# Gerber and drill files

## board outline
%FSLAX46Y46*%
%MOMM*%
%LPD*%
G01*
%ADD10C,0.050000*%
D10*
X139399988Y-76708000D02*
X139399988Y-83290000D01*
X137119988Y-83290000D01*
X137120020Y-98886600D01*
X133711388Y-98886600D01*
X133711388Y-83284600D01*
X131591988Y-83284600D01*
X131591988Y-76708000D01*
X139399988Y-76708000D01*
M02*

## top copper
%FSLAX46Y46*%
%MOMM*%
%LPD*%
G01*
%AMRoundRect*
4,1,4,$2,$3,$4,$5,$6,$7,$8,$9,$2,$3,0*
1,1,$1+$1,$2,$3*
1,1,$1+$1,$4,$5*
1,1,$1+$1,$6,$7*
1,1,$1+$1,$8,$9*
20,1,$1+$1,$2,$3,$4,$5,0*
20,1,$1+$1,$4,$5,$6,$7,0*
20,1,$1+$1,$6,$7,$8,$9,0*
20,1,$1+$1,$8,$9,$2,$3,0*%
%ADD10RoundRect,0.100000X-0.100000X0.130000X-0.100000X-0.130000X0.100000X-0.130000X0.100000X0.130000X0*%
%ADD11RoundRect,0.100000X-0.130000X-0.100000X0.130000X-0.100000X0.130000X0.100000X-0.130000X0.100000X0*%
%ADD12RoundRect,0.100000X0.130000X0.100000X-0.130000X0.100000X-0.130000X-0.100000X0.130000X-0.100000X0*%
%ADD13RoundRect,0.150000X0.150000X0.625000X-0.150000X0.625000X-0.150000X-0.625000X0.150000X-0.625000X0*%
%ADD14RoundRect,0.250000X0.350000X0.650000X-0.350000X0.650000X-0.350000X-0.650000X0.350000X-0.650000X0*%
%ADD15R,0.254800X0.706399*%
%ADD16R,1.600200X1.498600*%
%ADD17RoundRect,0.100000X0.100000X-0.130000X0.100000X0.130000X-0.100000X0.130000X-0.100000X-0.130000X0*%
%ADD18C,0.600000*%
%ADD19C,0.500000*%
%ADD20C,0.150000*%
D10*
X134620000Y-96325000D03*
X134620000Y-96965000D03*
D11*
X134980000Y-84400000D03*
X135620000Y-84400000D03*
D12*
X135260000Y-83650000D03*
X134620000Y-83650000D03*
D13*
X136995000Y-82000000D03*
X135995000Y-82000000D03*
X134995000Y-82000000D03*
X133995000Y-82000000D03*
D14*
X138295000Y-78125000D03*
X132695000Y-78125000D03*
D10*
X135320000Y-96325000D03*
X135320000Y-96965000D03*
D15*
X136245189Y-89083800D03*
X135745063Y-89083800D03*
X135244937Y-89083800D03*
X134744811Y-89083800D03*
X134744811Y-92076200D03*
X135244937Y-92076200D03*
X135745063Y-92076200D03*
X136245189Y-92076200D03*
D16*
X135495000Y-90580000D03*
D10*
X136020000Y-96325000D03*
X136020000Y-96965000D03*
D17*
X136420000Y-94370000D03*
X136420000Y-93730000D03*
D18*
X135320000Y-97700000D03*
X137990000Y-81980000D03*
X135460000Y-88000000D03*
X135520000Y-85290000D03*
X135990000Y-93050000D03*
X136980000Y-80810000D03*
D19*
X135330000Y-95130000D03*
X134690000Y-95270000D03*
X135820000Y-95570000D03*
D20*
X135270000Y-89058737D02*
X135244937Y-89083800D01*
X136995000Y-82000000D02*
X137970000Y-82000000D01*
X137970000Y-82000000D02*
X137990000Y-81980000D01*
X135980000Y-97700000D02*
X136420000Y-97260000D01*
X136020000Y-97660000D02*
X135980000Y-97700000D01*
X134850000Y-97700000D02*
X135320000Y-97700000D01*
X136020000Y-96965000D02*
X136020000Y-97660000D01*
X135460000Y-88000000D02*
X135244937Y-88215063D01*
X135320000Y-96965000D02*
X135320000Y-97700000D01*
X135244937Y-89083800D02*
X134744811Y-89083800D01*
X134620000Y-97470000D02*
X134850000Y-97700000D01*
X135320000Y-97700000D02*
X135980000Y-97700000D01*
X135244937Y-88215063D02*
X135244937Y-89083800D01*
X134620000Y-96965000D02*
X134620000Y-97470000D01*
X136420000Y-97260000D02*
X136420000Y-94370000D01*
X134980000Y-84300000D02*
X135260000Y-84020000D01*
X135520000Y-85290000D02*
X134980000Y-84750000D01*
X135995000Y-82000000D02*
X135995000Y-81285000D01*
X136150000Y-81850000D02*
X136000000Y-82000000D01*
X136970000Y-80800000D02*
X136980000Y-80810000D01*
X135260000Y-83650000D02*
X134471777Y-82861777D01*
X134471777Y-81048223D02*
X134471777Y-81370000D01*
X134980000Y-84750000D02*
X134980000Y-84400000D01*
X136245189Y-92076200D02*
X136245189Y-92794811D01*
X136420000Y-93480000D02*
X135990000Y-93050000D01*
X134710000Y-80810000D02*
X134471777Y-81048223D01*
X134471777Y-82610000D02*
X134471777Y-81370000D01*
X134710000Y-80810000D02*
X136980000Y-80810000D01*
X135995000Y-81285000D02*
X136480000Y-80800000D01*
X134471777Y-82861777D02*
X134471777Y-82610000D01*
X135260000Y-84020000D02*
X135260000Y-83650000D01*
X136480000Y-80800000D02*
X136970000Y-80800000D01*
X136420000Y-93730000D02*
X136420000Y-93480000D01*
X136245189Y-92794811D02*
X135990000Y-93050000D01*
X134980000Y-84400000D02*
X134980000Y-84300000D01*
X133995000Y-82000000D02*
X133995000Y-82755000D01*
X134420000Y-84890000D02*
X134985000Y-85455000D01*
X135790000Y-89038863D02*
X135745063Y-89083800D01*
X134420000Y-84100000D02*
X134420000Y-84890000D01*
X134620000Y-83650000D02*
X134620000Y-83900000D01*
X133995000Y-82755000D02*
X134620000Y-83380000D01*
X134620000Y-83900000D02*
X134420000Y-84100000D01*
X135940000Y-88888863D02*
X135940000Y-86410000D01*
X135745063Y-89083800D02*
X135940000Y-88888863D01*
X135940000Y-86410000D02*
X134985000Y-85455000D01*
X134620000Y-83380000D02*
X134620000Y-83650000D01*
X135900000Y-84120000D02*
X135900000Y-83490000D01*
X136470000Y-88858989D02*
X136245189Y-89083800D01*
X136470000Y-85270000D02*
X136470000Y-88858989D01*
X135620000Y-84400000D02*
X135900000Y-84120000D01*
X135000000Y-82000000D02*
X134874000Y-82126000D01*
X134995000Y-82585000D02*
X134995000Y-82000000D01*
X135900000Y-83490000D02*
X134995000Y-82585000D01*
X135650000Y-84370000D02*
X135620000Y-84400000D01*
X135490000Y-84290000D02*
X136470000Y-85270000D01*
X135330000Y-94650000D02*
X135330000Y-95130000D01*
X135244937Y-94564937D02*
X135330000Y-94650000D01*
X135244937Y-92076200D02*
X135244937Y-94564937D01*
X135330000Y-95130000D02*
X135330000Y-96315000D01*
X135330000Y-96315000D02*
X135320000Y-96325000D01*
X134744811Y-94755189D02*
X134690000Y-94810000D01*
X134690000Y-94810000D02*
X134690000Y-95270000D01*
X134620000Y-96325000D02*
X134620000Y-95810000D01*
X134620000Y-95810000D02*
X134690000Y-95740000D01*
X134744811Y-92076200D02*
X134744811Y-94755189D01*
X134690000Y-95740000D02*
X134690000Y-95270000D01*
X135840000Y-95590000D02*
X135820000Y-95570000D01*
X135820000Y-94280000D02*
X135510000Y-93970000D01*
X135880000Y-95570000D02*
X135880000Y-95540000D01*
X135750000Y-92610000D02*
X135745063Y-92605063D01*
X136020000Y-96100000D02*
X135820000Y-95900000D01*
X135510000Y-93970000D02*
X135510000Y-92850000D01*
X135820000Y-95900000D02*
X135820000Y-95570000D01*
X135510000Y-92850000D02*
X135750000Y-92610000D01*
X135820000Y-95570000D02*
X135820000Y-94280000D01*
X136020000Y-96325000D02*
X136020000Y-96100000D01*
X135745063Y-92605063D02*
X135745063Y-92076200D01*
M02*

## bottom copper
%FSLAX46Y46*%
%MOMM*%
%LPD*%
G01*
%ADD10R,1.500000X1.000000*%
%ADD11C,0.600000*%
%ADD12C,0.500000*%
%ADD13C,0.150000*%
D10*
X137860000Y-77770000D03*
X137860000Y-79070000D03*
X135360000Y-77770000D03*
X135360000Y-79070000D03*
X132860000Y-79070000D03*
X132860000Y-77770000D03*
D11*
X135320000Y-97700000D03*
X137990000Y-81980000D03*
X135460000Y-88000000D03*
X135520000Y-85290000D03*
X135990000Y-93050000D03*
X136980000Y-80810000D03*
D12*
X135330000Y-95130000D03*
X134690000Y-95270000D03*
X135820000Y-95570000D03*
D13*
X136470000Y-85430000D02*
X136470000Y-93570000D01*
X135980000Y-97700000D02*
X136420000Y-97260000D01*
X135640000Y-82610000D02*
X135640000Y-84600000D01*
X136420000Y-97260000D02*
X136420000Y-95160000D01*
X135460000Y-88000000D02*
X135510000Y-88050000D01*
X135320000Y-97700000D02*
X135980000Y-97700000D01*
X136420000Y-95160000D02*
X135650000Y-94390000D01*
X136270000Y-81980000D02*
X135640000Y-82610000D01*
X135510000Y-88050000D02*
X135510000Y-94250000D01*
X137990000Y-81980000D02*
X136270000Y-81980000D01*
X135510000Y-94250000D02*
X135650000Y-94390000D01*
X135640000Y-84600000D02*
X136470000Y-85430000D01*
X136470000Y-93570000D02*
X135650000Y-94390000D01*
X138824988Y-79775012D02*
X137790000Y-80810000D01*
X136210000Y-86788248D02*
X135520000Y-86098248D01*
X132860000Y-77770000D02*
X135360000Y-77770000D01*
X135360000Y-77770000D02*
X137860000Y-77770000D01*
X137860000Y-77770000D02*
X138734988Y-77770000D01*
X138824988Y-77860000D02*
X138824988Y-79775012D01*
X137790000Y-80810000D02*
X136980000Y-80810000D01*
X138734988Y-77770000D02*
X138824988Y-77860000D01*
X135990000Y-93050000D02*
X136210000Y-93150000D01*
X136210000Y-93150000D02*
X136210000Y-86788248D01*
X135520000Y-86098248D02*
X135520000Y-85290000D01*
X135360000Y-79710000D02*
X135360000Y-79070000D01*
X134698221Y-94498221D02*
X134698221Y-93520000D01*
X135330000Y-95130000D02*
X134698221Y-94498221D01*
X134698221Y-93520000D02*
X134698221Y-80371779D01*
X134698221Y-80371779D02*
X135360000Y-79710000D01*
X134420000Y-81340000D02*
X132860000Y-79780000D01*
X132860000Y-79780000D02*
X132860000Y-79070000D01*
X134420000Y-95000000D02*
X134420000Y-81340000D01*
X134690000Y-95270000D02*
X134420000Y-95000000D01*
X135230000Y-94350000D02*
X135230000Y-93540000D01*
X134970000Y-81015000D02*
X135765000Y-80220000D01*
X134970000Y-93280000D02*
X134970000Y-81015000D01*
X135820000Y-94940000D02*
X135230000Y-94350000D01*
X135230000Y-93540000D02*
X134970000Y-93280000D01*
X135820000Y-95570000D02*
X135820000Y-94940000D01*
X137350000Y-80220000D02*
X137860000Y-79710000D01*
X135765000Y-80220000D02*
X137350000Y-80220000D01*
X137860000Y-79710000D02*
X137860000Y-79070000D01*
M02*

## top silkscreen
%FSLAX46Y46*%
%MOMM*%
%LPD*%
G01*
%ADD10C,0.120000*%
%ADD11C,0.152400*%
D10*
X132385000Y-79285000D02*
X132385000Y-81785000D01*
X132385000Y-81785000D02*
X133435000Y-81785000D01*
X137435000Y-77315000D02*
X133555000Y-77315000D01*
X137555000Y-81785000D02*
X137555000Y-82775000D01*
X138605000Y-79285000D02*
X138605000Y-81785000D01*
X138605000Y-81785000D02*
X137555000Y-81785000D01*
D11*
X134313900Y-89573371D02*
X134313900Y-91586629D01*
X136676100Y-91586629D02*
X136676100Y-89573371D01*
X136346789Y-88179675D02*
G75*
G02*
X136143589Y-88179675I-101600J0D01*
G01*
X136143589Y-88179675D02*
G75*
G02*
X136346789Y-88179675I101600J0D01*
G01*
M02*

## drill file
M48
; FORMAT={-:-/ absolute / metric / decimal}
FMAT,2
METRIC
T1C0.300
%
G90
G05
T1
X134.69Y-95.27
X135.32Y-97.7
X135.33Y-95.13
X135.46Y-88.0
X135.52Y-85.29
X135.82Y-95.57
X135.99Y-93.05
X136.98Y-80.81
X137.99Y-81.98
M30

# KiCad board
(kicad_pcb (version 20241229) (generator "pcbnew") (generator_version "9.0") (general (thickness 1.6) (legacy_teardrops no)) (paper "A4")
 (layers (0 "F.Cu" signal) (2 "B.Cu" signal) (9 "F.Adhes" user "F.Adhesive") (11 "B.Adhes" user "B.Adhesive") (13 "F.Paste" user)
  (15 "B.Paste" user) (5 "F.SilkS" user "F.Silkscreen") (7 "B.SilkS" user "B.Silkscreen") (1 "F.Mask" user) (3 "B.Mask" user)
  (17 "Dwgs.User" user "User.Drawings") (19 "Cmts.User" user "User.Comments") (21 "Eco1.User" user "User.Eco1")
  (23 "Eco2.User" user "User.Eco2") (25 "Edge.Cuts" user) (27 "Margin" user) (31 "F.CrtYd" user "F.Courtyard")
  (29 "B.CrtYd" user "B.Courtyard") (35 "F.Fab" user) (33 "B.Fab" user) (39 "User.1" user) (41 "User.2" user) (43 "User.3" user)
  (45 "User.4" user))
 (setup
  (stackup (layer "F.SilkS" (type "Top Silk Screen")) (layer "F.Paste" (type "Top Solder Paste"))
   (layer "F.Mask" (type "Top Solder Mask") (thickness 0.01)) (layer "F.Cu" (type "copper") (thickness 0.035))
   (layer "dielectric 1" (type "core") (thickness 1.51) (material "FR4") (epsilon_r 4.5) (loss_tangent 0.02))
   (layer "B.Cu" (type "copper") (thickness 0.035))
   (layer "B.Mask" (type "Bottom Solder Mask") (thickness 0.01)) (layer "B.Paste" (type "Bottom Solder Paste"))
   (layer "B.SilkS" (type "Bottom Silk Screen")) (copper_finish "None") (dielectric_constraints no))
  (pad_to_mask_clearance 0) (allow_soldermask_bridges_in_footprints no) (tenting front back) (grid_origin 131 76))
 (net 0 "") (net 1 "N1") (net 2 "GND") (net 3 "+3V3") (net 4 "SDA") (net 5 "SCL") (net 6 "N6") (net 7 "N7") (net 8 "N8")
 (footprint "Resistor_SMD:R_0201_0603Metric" (layer "F.Cu") (at 134.62 96.645 -90)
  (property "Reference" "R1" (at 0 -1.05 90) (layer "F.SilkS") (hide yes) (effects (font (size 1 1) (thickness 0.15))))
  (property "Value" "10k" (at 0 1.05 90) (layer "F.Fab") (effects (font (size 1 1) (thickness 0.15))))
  (pad "" smd roundrect (at -0.345 0 270) (size 0.318 0.36) (layers "F.Paste") (roundrect_rratio 0.25))
  (pad "" smd roundrect (at 0.345 0 270) (size 0.318 0.36) (layers "F.Paste") (roundrect_rratio 0.25))
  (pad "1" smd roundrect (at -0.32 0 270) (size 0.46 0.4) (layers "F.Cu" "F.Mask") (roundrect_rratio 0.25) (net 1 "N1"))
  (pad "2" smd roundrect (at 0.32 0 270) (size 0.46 0.4) (layers "F.Cu" "F.Mask") (roundrect_rratio 0.25) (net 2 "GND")))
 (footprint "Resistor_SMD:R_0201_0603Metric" (layer "F.Cu") (at 135.3 84.4)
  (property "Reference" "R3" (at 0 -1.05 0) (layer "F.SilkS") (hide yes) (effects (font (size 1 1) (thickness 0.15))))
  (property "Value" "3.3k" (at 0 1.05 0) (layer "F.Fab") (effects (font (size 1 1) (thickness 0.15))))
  (pad "" smd roundrect (at -0.345 0) (size 0.318 0.36) (layers "F.Paste") (roundrect_rratio 0.25))
  (pad "" smd roundrect (at 0.345 0) (size 0.318 0.36) (layers "F.Paste") (roundrect_rratio 0.25))
  (pad "1" smd roundrect (at -0.32 0) (size 0.46 0.4) (layers "F.Cu" "F.Mask") (roundrect_rratio 0.25) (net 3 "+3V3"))
  (pad "2" smd roundrect (at 0.32 0) (size 0.46 0.4) (layers "F.Cu" "F.Mask") (roundrect_rratio 0.25) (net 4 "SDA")))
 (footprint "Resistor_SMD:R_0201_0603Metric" (layer "F.Cu") (at 134.94 83.65 180)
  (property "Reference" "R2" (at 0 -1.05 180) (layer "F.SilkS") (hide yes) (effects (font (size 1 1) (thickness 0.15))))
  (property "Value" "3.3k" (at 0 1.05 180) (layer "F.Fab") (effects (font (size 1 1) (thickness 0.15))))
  (pad "" smd roundrect (at -0.345 0 180) (size 0.318 0.36) (layers "F.Paste") (roundrect_rratio 0.25))
  (pad "" smd roundrect (at 0.345 0 180) (size 0.318 0.36) (layers "F.Paste") (roundrect_rratio 0.25))
  (pad "1" smd roundrect (at -0.32 0 180) (size 0.46 0.4) (layers "F.Cu" "F.Mask") (roundrect_rratio 0.25) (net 3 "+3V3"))
  (pad "2" smd roundrect (at 0.32 0 180) (size 0.46 0.4) (layers "F.Cu" "F.Mask") (roundrect_rratio 0.25) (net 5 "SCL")))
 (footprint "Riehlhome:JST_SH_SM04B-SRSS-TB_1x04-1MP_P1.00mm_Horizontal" (layer "F.Cu") (at 135.495 80 180)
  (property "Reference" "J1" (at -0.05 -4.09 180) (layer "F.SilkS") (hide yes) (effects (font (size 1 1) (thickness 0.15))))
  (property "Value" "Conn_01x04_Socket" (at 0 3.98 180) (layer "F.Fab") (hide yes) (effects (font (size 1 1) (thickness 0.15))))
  (fp_line (start 3.11 0.715) (end 3.11 -1.785) (stroke (width 0.12) (type solid)) (layer "F.SilkS"))
  (fp_line (start 3.11 -1.785) (end 2.06 -1.785) (stroke (width 0.12) (type solid)) (layer "F.SilkS"))
  (fp_line (start -1.94 2.685) (end 1.94 2.685) (stroke (width 0.12) (type solid)) (layer "F.SilkS"))
  (fp_line (start -2.06 -1.785) (end -2.06 -2.775) (stroke (width 0.12) (type solid)) (layer "F.SilkS"))
  (fp_line (start -3.11 0.715) (end -3.11 -1.785) (stroke (width 0.12) (type solid)) (layer "F.SilkS"))
  (fp_line (start -3.11 -1.785) (end -2.06 -1.785) (stroke (width 0.12) (type solid)) (layer "F.SilkS"))
  (pad "1" smd roundrect (at -1.5 -2 180) (size 0.6 1.55) (layers "F.Cu" "F.Mask" "F.Paste") (roundrect_rratio 0.25) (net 2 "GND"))
  (pad "2" smd roundrect (at -0.5 -2 180) (size 0.6 1.55) (layers "F.Cu" "F.Mask" "F.Paste") (roundrect_rratio 0.25) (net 3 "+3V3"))
  (pad "3" smd roundrect (at 0.5 -2 180) (size 0.6 1.55) (layers "F.Cu" "F.Mask" "F.Paste") (roundrect_rratio 0.25) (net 4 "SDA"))
  (pad "4" smd roundrect (at 1.5 -2 180) (size 0.6 1.55) (layers "F.Cu" "F.Mask" "F.Paste") (roundrect_rratio 0.25) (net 5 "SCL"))
  (pad "MP" smd roundrect (at -2.8 1.875 180) (size 1.2 1.8) (layers "F.Cu" "F.Mask" "F.Paste") (roundrect_rratio 0.208333))
  (pad "MP" smd roundrect (at 2.8 1.875 180) (size 1.2 1.8) (layers "F.Cu" "F.Mask" "F.Paste") (roundrect_rratio 0.208333)))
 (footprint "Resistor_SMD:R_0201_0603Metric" (layer "F.Cu") (at 135.32 96.645 -90)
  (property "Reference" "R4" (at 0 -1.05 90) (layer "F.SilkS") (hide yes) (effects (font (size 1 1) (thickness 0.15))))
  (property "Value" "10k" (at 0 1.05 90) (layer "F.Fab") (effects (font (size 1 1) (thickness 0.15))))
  (pad "" smd roundrect (at -0.345 0 270) (size 0.318 0.36) (layers "F.Paste") (roundrect_rratio 0.25))
  (pad "" smd roundrect (at 0.345 0 270) (size 0.318 0.36) (layers "F.Paste") (roundrect_rratio 0.25))
  (pad "1" smd roundrect (at -0.32 0 270) (size 0.46 0.4) (layers "F.Cu" "F.Mask") (roundrect_rratio 0.25) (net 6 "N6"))
  (pad "2" smd roundrect (at 0.32 0 270) (size 0.46 0.4) (layers "F.Cu" "F.Mask") (roundrect_rratio 0.25) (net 2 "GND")))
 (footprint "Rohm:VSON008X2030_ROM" (layer "F.Cu") (at 135.495 90.58 -90)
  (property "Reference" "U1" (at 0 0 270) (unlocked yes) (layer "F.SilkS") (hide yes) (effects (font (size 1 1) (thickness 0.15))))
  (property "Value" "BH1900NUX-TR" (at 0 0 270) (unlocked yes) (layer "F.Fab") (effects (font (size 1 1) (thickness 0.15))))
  (fp_line (start -1.006629 1.1811) (end 1.006629 1.1811) (stroke (width 0.1524) (type solid)) (layer "F.SilkS"))
  (fp_line (start 1.006629 -1.1811) (end -1.006629 -1.1811) (stroke (width 0.1524) (type solid)) (layer "F.SilkS"))
  (fp_circle (center -2.400325 -0.750189) (end -2.298725 -0.750189) (stroke (width 0.1524) (type solid)) (fill no) (layer "F.SilkS"))
  (pad "1" smd rect (at -1.4962 -0.750189 270) (size 0.706399 0.2548) (layers "F.Cu" "F.Mask" "F.Paste") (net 4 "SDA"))
  (pad "2" smd rect (at -1.4962 -0.250063 270) (size 0.706399 0.2548) (layers "F.Cu" "F.Mask" "F.Paste") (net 5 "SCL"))
  (pad "3" smd rect (at -1.4962 0.250063 270) (size 0.706399 0.2548) (layers "F.Cu" "F.Mask" "F.Paste") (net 2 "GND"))
  (pad "4" smd rect (at -1.4962 0.750189 270) (size 0.706399 0.2548) (layers "F.Cu" "F.Mask" "F.Paste") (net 2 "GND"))
  (pad "5" smd rect (at 1.4962 0.750189 270) (size 0.706399 0.2548) (layers "F.Cu" "F.Mask" "F.Paste") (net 1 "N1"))
  (pad "6" smd rect (at 1.4962 0.250063 270) (size 0.706399 0.2548) (layers "F.Cu" "F.Mask" "F.Paste") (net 6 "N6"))
  (pad "7" smd rect (at 1.4962 -0.250063 270) (size 0.706399 0.2548) (layers "F.Cu" "F.Mask" "F.Paste") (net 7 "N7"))
  (pad "8" smd rect (at 1.4962 -0.750189 270) (size 0.706399 0.2548) (layers "F.Cu" "F.Mask" "F.Paste") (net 3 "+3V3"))
  (pad "9" smd rect (at 0 0 270) (size 1.4986 1.6002) (layers "F.Cu" "F.Mask" "F.Paste") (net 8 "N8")))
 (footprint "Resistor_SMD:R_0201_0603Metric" (layer "F.Cu") (at 136.02 96.645 -90)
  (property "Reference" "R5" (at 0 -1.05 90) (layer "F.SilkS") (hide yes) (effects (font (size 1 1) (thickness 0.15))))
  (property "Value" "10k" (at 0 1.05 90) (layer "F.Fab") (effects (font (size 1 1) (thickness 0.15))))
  (pad "" smd roundrect (at -0.345 0 270) (size 0.318 0.36) (layers "F.Paste") (roundrect_rratio 0.25))
  (pad "" smd roundrect (at 0.345 0 270) (size 0.318 0.36) (layers "F.Paste") (roundrect_rratio 0.25))
  (pad "1" smd roundrect (at -0.32 0 270) (size 0.46 0.4) (layers "F.Cu" "F.Mask") (roundrect_rratio 0.25) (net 7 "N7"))
  (pad "2" smd roundrect (at 0.32 0 270) (size 0.46 0.4) (layers "F.Cu" "F.Mask") (roundrect_rratio 0.25) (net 2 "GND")))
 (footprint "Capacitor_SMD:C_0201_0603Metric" (layer "F.Cu") (at 136.42 94.05 90)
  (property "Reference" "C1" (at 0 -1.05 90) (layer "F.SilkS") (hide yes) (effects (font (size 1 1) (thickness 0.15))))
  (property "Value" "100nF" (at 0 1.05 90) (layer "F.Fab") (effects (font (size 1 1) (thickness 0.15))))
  (pad "" smd roundrect (at -0.345 0 90) (size 0.318 0.36) (layers "F.Paste") (roundrect_rratio 0.25))
  (pad "" smd roundrect (at 0.345 0 90) (size 0.318 0.36) (layers "F.Paste") (roundrect_rratio 0.25))
  (pad "1" smd roundrect (at -0.32 0 90) (size 0.46 0.4) (layers "F.Cu" "F.Mask") (roundrect_rratio 0.25) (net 2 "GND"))
  (pad "2" smd roundrect (at 0.32 0 90) (size 0.46 0.4) (layers "F.Cu" "F.Mask") (roundrect_rratio 0.25) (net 3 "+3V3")))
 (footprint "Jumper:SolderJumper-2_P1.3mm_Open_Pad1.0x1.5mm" (layer "B.Cu") (at 137.86 78.42 -90)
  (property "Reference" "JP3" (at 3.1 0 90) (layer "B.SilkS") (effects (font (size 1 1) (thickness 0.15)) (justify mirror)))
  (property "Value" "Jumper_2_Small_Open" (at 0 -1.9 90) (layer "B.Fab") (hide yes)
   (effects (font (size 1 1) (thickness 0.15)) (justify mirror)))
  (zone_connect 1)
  (pad "1" smd rect (at -0.65 0 270) (size 1 1.5) (layers "B.Cu" "B.Mask") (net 3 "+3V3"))
  (pad "2" smd rect (at 0.65 0 270) (size 1 1.5) (layers "B.Cu" "B.Mask") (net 7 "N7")))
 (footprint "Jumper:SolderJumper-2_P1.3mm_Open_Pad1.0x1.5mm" (layer "B.Cu") (at 135.36 78.42 -90)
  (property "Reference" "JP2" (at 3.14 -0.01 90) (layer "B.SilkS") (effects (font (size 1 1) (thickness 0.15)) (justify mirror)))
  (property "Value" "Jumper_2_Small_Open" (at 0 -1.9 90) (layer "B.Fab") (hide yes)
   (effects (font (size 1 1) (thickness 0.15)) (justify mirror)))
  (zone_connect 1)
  (pad "1" smd rect (at -0.65 0 270) (size 1 1.5) (layers "B.Cu" "B.Mask") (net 3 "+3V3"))
  (pad "2" smd rect (at 0.65 0 270) (size 1 1.5) (layers "B.Cu" "B.Mask") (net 6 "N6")))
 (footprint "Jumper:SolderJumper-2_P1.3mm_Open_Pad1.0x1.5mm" (layer "B.Cu") (at 132.86 78.42 90)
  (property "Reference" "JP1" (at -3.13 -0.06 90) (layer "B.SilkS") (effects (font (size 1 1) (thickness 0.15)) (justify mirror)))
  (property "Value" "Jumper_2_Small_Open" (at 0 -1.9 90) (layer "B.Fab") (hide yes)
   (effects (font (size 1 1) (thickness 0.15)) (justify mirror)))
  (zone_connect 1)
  (pad "1" smd rect (at -0.65 0 90) (size 1 1.5) (layers "B.Cu" "B.Mask") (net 1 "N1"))
  (pad "2" smd rect (at 0.65 0 90) (size 1 1.5) (layers "B.Cu" "B.Mask") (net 3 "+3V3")))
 (gr_poly
  (pts (xy 139.399988 76.708) (xy 139.399988 83.29) (xy 137.119988 83.29) (xy 137.12002 98.8866) (xy 133.711388 98.8866)
   (xy 133.711388 83.2846) (xy 131.591988 83.2846) (xy 131.591988 76.708))
  (stroke (width 0.05) (type solid)) (fill no) (layer "Edge.Cuts"))
 (segment (start 135.27 89.058737) (end 135.244937 89.0838) (width 0.15) (layer "F.Cu") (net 2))
 (segment (start 136.995 82) (end 137.97 82) (width 0.15) (layer "F.Cu") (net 2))
 (segment (start 137.97 82) (end 137.99 81.98) (width 0.15) (layer "F.Cu") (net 2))
 (segment (start 135.98 97.7) (end 136.42 97.26) (width 0.15) (layer "F.Cu") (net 2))
 (segment (start 136.02 97.66) (end 135.98 97.7) (width 0.15) (layer "F.Cu") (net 2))
 (segment (start 134.85 97.7) (end 135.32 97.7) (width 0.15) (layer "F.Cu") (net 2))
 (segment (start 136.02 96.965) (end 136.02 97.66) (width 0.15) (layer "F.Cu") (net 2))
 (segment (start 135.46 88) (end 135.244937 88.215063) (width 0.15) (layer "F.Cu") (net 2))
 (segment (start 135.32 96.965) (end 135.32 97.7) (width 0.15) (layer "F.Cu") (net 2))
 (segment (start 135.244937 89.0838) (end 134.744811 89.0838) (width 0.15) (layer "F.Cu") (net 2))
 (segment (start 134.62 97.47) (end 134.85 97.7) (width 0.15) (layer "F.Cu") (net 2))
 (segment (start 135.32 97.7) (end 135.98 97.7) (width 0.15) (layer "F.Cu") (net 2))
 (segment (start 135.244937 88.215063) (end 135.244937 89.0838) (width 0.15) (layer "F.Cu") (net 2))
 (segment (start 134.62 96.965) (end 134.62 97.47) (width 0.15) (layer "F.Cu") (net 2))
 (segment (start 136.42 97.26) (end 136.42 94.37) (width 0.15) (layer "F.Cu") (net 2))
 (via (at 135.32 97.7) (size 0.6) (drill 0.3) (layers "F.Cu" "B.Cu") (free yes) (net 2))
 (via (at 137.99 81.98) (size 0.6) (drill 0.3) (layers "F.Cu" "B.Cu") (free yes) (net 2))
 (via (at 135.46 88) (size 0.6) (drill 0.3) (layers "F.Cu" "B.Cu") (free yes) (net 2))
 (segment (start 136.47 85.43) (end 136.47 93.57) (width 0.15) (layer "B.Cu") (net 2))
 (segment (start 135.98 97.7) (end 136.42 97.26) (width 0.15) (layer "B.Cu") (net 2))
 (segment (start 135.64 82.61) (end 135.64 84.6) (width 0.15) (layer "B.Cu") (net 2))
 (segment (start 136.42 97.26) (end 136.42 95.16) (width 0.15) (layer "B.Cu") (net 2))
 (segment (start 135.46 88) (end 135.51 88.05) (width 0.15) (layer "B.Cu") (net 2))
 (segment (start 135.32 97.7) (end 135.98 97.7) (width 0.15) (layer "B.Cu") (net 2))
 (segment (start 136.42 95.16) (end 135.65 94.39) (width 0.15) (layer "B.Cu") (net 2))
 (segment (start 136.27 81.98) (end 135.64 82.61) (width 0.15) (layer "B.Cu") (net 2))
 (segment (start 135.51 88.05) (end 135.51 94.25) (width 0.15) (layer "B.Cu") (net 2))
 (segment (start 137.99 81.98) (end 136.27 81.98) (width 0.15) (layer "B.Cu") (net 2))
 (segment (start 135.51 94.25) (end 135.65 94.39) (width 0.15) (layer "B.Cu") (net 2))
 (segment (start 135.64 84.6) (end 136.47 85.43) (width 0.15) (layer "B.Cu") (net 2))
 (segment (start 136.47 93.57) (end 135.65 94.39) (width 0.15) (layer "B.Cu") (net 2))
 (segment (start 134.98 84.3) (end 135.26 84.02) (width 0.15) (layer "F.Cu") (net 3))
 (segment (start 135.52 85.29) (end 134.98 84.75) (width 0.15) (layer "F.Cu") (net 3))
 (segment (start 135.995 82) (end 135.995 81.285) (width 0.15) (layer "F.Cu") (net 3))
 (segment (start 136.15 81.85) (end 136 82) (width 0.15) (layer "F.Cu") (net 3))
 (segment (start 136.97 80.8) (end 136.98 80.81) (width 0.15) (layer "F.Cu") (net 3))
 (segment (start 135.26 83.65) (end 134.471777 82.861777) (width 0.15) (layer "F.Cu") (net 3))
 (segment (start 134.471777 81.048223) (end 134.471777 81.37) (width 0.15) (layer "F.Cu") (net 3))
 (segment (start 134.98 84.75) (end 134.98 84.4) (width 0.15) (layer "F.Cu") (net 3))
 (segment (start 136.245189 92.0762) (end 136.245189 92.794811) (width 0.15) (layer "F.Cu") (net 3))
 (segment (start 136.42 93.48) (end 135.99 93.05) (width 0.15) (layer "F.Cu") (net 3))
 (segment (start 134.71 80.81) (end 134.471777 81.048223) (width 0.15) (layer "F.Cu") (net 3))
 (segment (start 134.471777 82.61) (end 134.471777 81.37) (width 0.15) (layer "F.Cu") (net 3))
 (segment (start 134.71 80.81) (end 136.98 80.81) (width 0.15) (layer "F.Cu") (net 3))
 (segment (start 135.995 81.285) (end 136.48 80.8) (width 0.15) (layer "F.Cu") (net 3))
 (segment (start 134.471777 82.861777) (end 134.471777 82.61) (width 0.15) (layer "F.Cu") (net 3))
 (segment (start 135.26 84.02) (end 135.26 83.65) (width 0.15) (layer "F.Cu") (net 3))
 (segment (start 136.48 80.8) (end 136.97 80.8) (width 0.15) (layer "F.Cu") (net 3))
 (segment (start 136.42 93.73) (end 136.42 93.48) (width 0.15) (layer "F.Cu") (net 3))
 (segment (start 136.245189 92.794811) (end 135.99 93.05) (width 0.15) (layer "F.Cu") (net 3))
 (segment (start 134.98 84.4) (end 134.98 84.3) (width 0.15) (layer "F.Cu") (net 3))
 (via (at 135.52 85.29) (size 0.6) (drill 0.3) (layers "F.Cu" "B.Cu") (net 3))
 (via (at 135.99 93.05) (size 0.6) (drill 0.3) (layers "F.Cu" "B.Cu") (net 3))
 (via (at 136.98 80.81) (size 0.6) (drill 0.3) (layers "F.Cu" "B.Cu") (free yes) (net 3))
 (segment (start 138.824988 79.775012) (end 137.79 80.81) (width 0.15) (layer "B.Cu") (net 3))
 (segment (start 136.21 86.788248) (end 135.52 86.098248) (width 0.15) (layer "B.Cu") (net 3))
 (segment (start 132.86 77.77) (end 135.36 77.77) (width 0.15) (layer "B.Cu") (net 3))
 (segment (start 135.36 77.77) (end 137.86 77.77) (width 0.15) (layer "B.Cu") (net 3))
 (segment (start 137.86 77.77) (end 138.734988 77.77) (width 0.15) (layer "B.Cu") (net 3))
 (segment (start 138.824988 77.86) (end 138.824988 79.775012) (width 0.15) (layer "B.Cu") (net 3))
 (segment (start 137.79 80.81) (end 136.98 80.81) (width 0.15) (layer "B.Cu") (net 3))
 (segment (start 138.734988 77.77) (end 138.824988 77.86) (width 0.15) (layer "B.Cu") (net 3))
 (segment (start 135.99 93.05) (end 136.21 93.15) (width 0.15) (layer "B.Cu") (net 3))
 (segment (start 136.21 93.15) (end 136.21 86.788248) (width 0.15) (layer "B.Cu") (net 3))
 (segment (start 135.52 86.098248) (end 135.52 85.29) (width 0.15) (layer "B.Cu") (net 3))
 (segment (start 133.995 82) (end 133.995 82.755) (width 0.15) (layer "F.Cu") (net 5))
 (segment (start 134.42 84.89) (end 134.985 85.455) (width 0.15) (layer "F.Cu") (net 5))
 (segment (start 135.79 89.038863) (end 135.745063 89.0838) (width 0.15) (layer "F.Cu") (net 5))
 (segment (start 134.42 84.1) (end 134.42 84.89) (width 0.15) (layer "F.Cu") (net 5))
 (segment (start 134.62 83.65) (end 134.62 83.9) (width 0.15) (layer "F.Cu") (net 5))
 (segment (start 133.995 82.755) (end 134.62 83.38) (width 0.15) (layer "F.Cu") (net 5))
 (segment (start 134.62 83.9) (end 134.42 84.1) (width 0.15) (layer "F.Cu") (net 5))
 (segment (start 135.94 88.888863) (end 135.94 86.41) (width 0.15) (layer "F.Cu") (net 5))
 (segment (start 135.745063 89.0838) (end 135.94 88.888863) (width 0.15) (layer "F.Cu") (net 5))
 (segment (start 135.94 86.41) (end 134.985 85.455) (width 0.15) (layer "F.Cu") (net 5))
 (segment (start 134.62 83.38) (end 134.62 83.65) (width 0.15) (layer "F.Cu") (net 5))
 (segment (start 135.9 84.12) (end 135.9 83.49) (width 0.15) (layer "F.Cu") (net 4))
 (segment (start 136.47 88.858989) (end 136.245189 89.0838) (width 0.15) (layer "F.Cu") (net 4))
 (segment (start 136.47 85.27) (end 136.47 88.858989) (width 0.15) (layer "F.Cu") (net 4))
 (segment (start 135.62 84.4) (end 135.9 84.12) (width 0.15) (layer "F.Cu") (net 4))
 (segment (start 135 82) (end 134.874 82.126) (width 0.15) (layer "F.Cu") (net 4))
 (segment (start 134.995 82.585) (end 134.995 82) (width 0.15) (layer "F.Cu") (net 4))
 (segment (start 135.9 83.49) (end 134.995 82.585) (width 0.15) (layer "F.Cu") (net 4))
 (segment (start 135.65 84.37) (end 135.62 84.4) (width 0.15) (layer "F.Cu") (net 4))
 (segment (start 135.49 84.29) (end 136.47 85.27) (width 0.15) (layer "F.Cu") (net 4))
 (segment (start 135.33 94.65) (end 135.33 95.13) (width 0.15) (layer "F.Cu") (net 6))
 (segment (start 135.244937 94.564937) (end 135.33 94.65) (width 0.15) (layer "F.Cu") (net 6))
 (segment (start 135.244937 92.0762) (end 135.244937 94.564937) (width 0.15) (layer "F.Cu") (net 6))
 (segment (start 135.33 95.13) (end 135.33 96.315) (width 0.15) (layer "F.Cu") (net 6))
 (segment (start 135.33 96.315) (end 135.32 96.325) (width 0.15) (layer "F.Cu") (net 6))
 (via (at 135.33 95.13) (size 0.5) (drill 0.3) (layers "F.Cu" "B.Cu") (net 6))
 (segment (start 135.36 79.71) (end 135.36 79.07) (width 0.15) (layer "B.Cu") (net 6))
 (segment (start 134.698221 94.498221) (end 134.698221 93.52) (width 0.15) (layer "B.Cu") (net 6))
 (segment (start 135.33 95.13) (end 134.698221 94.498221) (width 0.15) (layer "B.Cu") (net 6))
 (segment (start 134.698221 93.52) (end 134.698221 80.371779) (width 0.15) (layer "B.Cu") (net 6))
 (segment (start 134.698221 80.371779) (end 135.36 79.71) (width 0.15) (layer "B.Cu") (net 6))
 (segment (start 134.744811 94.755189) (end 134.69 94.81) (width 0.15) (layer "F.Cu") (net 1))
 (segment (start 134.69 94.81) (end 134.69 95.27) (width 0.15) (layer "F.Cu") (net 1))
 (segment (start 134.62 96.325) (end 134.62 95.81) (width 0.15) (layer "F.Cu") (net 1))
 (segment (start 134.62 95.81) (end 134.69 95.74) (width 0.15) (layer "F.Cu") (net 1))
 (segment (start 134.744811 92.0762) (end 134.744811 94.755189) (width 0.15) (layer "F.Cu") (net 1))
 (segment (start 134.69 95.74) (end 134.69 95.27) (width 0.15) (layer "F.Cu") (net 1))
 (via (at 134.69 95.27) (size 0.5) (drill 0.3) (layers "F.Cu" "B.Cu") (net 1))
 (segment (start 134.42 81.34) (end 132.86 79.78) (width 0.15) (layer "B.Cu") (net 1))
 (segment (start 132.86 79.78) (end 132.86 79.07) (width 0.15) (layer "B.Cu") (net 1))
 (segment (start 134.42 95) (end 134.42 81.34) (width 0.15) (layer "B.Cu") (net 1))
 (segment (start 134.69 95.27) (end 134.42 95) (width 0.15) (layer "B.Cu") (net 1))
 (segment (start 135.84 95.59) (end 135.82 95.57) (width 0.15) (layer "F.Cu") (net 7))
 (segment (start 135.82 94.28) (end 135.51 93.97) (width 0.15) (layer "F.Cu") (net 7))
 (segment (start 135.88 95.57) (end 135.88 95.54) (width 0.15) (layer "F.Cu") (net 7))
 (segment (start 135.75 92.61) (end 135.745063 92.605063) (width 0.15) (layer "F.Cu") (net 7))
 (segment (start 136.02 96.1) (end 135.82 95.9) (width 0.15) (layer "F.Cu") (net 7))
 (segment (start 135.51 93.97) (end 135.51 92.85) (width 0.15) (layer "F.Cu") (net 7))
 (segment (start 135.82 95.9) (end 135.82 95.57) (width 0.15) (layer "F.Cu") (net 7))
 (segment (start 135.51 92.85) (end 135.75 92.61) (width 0.15) (layer "F.Cu") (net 7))
 (segment (start 135.82 95.57) (end 135.82 94.28) (width 0.15) (layer "F.Cu") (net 7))
 (segment (start 136.02 96.325) (end 136.02 96.1) (width 0.15) (layer "F.Cu") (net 7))
 (segment (start 135.745063 92.605063) (end 135.745063 92.0762) (width 0.15) (layer "F.Cu") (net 7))
 (via (at 135.82 95.57) (size 0.5) (drill 0.3) (layers "F.Cu" "B.Cu") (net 7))
 (segment (start 135.23 94.35) (end 135.23 93.54) (width 0.15) (layer "B.Cu") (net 7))
 (segment (start 134.97 81.015) (end 135.765 80.22) (width 0.15) (layer "B.Cu") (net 7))
 (segment (start 134.97 93.28) (end 134.97 81.015) (width 0.15) (layer "B.Cu") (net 7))
 (segment (start 135.82 94.94) (end 135.23 94.35) (width 0.15) (layer "B.Cu") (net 7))
 (segment (start 135.23 93.54) (end 134.97 93.28) (width 0.15) (layer "B.Cu") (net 7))
 (segment (start 135.82 95.57) (end 135.82 94.94) (width 0.15) (layer "B.Cu") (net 7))
 (segment (start 137.35 80.22) (end 137.86 79.71) (width 0.15) (layer "B.Cu") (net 7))
 (segment (start 135.765 80.22) (end 137.35 80.22) (width 0.15) (layer "B.Cu") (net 7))
 (segment (start 137.86 79.71) (end 137.86 79.07) (width 0.15) (layer "B.Cu") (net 7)))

